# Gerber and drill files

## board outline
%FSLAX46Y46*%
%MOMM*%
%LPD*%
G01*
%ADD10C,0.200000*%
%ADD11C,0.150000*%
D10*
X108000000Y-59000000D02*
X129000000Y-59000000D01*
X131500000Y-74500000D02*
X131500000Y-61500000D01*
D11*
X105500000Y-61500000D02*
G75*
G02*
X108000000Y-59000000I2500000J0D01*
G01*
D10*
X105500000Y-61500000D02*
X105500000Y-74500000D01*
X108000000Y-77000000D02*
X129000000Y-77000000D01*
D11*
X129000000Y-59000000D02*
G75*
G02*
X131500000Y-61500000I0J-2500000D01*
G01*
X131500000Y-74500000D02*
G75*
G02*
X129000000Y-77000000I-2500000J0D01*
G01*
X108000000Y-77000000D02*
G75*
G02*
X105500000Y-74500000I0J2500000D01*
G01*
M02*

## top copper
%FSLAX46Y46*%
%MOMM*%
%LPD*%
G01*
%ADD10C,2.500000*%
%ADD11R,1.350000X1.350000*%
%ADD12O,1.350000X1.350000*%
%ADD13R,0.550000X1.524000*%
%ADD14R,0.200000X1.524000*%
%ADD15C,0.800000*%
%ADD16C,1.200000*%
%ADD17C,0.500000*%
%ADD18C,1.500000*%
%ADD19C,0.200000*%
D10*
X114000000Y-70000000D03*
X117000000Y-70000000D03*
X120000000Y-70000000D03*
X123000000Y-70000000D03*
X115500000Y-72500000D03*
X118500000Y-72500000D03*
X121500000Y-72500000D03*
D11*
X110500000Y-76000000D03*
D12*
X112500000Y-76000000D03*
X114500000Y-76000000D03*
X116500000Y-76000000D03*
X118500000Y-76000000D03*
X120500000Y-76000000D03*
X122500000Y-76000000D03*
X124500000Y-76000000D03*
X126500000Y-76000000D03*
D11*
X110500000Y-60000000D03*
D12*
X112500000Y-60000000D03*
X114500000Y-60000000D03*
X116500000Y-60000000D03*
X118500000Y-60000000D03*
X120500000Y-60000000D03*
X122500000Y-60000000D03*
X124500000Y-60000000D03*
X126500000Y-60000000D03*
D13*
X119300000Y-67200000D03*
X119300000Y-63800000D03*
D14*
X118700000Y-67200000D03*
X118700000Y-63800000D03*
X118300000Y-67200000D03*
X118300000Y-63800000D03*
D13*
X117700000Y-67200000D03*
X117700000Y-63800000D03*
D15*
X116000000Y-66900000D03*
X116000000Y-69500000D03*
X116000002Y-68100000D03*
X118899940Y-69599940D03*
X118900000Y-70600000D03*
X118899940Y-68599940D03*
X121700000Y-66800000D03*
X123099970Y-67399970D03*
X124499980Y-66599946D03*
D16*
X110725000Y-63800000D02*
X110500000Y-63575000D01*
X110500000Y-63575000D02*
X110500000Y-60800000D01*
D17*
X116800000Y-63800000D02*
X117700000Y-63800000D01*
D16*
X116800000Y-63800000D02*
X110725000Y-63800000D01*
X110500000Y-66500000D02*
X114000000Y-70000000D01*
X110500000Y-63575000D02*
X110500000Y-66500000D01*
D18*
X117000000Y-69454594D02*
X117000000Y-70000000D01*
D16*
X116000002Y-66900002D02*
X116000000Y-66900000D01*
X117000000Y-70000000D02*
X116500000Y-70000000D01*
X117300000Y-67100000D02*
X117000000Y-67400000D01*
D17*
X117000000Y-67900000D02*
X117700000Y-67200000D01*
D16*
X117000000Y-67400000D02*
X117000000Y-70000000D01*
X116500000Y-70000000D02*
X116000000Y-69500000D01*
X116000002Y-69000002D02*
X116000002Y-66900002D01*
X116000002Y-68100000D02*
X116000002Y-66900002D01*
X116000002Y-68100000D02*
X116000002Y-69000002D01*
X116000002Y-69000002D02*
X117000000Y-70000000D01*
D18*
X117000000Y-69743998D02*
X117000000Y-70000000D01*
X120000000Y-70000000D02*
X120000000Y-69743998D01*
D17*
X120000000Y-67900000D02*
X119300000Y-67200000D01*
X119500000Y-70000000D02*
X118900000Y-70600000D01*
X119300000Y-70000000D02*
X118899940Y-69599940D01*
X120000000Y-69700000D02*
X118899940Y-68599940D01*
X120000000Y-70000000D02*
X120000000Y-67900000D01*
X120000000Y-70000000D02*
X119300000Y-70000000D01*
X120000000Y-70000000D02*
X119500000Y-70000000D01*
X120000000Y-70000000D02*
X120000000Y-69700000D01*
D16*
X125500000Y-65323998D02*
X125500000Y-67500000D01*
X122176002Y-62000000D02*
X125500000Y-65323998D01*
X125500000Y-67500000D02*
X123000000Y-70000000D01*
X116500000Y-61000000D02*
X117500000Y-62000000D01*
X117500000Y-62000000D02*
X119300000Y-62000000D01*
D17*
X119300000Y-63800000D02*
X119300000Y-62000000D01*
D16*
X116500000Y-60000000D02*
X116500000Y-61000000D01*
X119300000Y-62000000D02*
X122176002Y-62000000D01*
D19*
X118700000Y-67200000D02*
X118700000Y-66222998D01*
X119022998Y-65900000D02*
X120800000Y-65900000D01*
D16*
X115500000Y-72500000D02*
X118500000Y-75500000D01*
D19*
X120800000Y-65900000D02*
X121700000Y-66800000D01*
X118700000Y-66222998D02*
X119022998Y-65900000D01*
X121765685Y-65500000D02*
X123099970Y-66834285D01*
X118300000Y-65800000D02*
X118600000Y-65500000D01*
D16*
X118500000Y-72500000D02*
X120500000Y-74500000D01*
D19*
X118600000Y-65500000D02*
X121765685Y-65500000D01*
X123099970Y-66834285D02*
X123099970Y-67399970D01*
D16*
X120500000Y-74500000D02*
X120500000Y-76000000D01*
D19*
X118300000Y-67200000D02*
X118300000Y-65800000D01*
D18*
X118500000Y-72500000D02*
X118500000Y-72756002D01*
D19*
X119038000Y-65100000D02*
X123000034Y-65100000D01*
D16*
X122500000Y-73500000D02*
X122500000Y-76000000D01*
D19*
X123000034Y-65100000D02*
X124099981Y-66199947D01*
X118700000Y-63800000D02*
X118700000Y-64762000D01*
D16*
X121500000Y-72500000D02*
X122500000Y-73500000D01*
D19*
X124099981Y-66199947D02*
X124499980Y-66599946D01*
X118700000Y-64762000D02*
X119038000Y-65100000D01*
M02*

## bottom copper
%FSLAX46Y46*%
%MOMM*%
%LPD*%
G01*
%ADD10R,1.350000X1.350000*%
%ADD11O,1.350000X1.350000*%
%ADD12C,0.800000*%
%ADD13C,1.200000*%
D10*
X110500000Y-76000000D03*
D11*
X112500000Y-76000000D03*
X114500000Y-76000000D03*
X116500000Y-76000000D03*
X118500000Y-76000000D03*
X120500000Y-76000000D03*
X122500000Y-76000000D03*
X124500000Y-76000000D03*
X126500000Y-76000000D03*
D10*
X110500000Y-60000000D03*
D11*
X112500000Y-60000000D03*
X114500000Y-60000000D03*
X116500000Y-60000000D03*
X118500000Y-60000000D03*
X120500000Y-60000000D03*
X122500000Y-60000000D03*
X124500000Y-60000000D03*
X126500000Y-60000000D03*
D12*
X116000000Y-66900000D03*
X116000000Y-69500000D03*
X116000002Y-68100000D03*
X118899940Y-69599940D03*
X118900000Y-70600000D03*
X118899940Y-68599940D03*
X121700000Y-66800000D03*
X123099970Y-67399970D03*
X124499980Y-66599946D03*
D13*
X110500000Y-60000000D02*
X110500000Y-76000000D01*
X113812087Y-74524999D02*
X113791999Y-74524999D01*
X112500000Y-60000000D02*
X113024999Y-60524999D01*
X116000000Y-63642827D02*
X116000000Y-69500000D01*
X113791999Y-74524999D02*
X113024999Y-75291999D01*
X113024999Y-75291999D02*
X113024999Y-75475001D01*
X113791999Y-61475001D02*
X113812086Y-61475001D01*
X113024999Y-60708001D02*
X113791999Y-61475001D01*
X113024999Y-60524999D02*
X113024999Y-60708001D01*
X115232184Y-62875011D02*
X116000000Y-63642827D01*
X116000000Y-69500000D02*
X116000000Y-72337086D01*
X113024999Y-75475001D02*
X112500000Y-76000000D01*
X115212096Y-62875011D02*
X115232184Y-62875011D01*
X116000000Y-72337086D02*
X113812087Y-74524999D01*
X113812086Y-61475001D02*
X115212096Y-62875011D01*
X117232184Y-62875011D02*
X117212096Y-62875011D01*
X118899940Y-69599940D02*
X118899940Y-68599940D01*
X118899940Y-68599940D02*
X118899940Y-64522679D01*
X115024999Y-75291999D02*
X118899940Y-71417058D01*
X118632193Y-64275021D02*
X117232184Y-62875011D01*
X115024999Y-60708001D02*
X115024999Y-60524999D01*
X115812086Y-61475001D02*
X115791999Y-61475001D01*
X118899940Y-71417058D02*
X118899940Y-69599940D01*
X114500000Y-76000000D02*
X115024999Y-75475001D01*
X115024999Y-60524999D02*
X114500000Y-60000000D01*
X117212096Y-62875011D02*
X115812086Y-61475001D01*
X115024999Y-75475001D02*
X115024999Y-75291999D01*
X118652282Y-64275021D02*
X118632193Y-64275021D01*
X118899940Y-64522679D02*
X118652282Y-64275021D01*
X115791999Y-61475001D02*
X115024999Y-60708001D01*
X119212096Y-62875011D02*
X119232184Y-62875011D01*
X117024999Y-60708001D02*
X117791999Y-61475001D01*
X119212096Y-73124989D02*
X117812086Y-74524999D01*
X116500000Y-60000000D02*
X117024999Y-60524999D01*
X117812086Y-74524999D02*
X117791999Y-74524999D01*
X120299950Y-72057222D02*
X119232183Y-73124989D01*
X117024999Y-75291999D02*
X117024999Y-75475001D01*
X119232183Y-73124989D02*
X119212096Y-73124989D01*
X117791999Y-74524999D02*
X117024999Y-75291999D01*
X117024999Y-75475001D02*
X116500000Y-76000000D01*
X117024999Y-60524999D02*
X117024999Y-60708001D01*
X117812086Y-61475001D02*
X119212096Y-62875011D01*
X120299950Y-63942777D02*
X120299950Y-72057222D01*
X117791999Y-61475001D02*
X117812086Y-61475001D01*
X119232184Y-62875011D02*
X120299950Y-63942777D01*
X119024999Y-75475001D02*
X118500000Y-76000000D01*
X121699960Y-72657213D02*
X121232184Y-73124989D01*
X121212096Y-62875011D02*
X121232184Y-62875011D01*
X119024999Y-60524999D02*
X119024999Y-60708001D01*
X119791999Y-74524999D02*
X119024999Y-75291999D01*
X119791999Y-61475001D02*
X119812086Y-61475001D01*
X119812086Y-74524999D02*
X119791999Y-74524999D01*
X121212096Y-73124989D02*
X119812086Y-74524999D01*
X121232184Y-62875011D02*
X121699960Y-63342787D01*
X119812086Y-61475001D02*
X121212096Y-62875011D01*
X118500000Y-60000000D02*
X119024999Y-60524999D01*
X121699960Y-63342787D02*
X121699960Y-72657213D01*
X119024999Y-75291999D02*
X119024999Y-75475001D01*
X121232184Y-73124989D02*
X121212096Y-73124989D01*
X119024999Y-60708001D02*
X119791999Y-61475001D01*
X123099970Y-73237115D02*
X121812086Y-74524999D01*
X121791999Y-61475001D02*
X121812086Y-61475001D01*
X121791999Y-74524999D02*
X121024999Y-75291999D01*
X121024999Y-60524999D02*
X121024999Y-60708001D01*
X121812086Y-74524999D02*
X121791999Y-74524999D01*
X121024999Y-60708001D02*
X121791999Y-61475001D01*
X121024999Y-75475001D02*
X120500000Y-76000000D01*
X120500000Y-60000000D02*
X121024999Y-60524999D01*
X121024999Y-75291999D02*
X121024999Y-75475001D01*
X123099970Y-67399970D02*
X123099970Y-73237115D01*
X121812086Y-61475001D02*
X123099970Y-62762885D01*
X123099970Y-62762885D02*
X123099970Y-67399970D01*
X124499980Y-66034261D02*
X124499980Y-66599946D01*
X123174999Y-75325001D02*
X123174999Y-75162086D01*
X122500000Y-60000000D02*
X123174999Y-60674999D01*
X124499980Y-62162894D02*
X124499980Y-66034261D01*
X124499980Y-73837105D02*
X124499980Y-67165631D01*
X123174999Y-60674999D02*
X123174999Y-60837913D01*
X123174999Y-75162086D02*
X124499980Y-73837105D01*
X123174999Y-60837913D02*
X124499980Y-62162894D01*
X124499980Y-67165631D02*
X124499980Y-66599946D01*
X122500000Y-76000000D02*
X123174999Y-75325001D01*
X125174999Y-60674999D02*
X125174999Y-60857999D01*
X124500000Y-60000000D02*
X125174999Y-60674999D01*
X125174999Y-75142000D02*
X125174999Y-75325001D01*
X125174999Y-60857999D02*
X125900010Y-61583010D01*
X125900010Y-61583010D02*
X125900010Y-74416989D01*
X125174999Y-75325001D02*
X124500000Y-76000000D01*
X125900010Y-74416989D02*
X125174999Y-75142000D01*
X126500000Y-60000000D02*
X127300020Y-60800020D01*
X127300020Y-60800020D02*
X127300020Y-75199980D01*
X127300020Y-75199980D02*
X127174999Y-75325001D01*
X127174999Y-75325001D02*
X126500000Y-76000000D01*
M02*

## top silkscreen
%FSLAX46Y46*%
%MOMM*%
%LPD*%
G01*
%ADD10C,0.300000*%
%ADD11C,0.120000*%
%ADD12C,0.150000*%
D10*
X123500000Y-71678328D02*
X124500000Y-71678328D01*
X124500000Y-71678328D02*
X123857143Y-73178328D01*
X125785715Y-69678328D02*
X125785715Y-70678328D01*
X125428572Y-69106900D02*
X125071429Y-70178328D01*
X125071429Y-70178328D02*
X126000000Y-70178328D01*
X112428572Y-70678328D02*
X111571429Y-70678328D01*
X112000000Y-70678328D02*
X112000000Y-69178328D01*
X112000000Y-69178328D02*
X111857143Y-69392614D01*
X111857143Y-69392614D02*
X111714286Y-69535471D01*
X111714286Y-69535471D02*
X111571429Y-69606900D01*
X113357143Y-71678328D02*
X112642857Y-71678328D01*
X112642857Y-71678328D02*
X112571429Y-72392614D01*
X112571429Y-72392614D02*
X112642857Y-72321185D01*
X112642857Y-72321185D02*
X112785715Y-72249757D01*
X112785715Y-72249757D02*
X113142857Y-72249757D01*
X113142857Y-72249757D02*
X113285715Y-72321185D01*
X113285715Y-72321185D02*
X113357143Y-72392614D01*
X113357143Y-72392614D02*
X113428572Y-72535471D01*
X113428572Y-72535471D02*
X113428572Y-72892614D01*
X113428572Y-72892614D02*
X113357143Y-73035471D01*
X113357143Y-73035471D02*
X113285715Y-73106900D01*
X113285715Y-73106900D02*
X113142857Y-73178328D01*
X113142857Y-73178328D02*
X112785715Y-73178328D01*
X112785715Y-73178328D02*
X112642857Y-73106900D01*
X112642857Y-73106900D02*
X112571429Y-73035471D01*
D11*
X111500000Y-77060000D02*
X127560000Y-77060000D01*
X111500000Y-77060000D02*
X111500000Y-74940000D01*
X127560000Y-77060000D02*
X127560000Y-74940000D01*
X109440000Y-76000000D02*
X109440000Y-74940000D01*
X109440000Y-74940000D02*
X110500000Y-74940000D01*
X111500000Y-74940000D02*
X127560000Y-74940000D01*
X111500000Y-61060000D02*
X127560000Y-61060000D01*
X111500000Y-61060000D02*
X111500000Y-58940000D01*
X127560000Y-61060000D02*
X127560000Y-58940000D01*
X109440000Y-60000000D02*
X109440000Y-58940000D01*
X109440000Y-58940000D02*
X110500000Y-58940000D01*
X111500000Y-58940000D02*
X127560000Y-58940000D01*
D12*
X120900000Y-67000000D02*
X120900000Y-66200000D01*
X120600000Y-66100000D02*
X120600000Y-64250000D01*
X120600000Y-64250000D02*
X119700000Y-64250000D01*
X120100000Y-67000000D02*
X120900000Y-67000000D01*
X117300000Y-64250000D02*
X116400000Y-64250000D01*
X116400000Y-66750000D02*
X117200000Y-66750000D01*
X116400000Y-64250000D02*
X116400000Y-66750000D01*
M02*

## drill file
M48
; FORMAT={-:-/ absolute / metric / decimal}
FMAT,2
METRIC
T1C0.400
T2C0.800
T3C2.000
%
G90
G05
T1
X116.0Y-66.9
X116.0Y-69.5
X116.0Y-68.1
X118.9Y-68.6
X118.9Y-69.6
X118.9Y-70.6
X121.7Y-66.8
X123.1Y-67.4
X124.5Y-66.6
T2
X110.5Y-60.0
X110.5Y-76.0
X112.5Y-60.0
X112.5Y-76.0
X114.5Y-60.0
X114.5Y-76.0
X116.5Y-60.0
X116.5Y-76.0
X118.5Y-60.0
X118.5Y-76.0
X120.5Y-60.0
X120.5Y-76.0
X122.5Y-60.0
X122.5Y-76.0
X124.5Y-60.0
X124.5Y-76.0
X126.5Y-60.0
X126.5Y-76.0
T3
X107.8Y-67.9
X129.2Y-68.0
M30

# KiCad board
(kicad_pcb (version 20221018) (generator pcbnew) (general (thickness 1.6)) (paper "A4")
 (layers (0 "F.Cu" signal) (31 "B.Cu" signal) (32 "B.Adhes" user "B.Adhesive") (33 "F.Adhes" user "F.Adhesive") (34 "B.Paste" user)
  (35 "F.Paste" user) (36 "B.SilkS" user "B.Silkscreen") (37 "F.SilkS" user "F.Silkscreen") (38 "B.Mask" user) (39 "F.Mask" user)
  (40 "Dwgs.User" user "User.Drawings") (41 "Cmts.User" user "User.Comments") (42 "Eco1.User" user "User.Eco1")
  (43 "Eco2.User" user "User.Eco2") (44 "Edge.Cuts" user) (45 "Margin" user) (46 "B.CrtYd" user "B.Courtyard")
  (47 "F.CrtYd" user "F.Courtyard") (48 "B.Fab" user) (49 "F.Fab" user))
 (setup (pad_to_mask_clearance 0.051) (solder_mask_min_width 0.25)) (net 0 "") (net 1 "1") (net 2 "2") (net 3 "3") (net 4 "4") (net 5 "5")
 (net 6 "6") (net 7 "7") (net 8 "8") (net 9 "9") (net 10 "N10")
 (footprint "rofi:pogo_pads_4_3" (layer "F.Cu") (at 118.5 70)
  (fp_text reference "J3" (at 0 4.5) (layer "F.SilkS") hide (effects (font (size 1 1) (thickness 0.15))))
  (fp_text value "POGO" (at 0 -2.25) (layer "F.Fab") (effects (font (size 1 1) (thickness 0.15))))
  (pad "1" smd circle (at -4.5 0) (size 2.5 2.5) (layers "F.Cu" "F.Paste" "F.Mask") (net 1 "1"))
  (pad "2" smd circle (at -1.5 0) (size 2.5 2.5) (layers "F.Cu" "F.Paste" "F.Mask") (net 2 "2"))
  (pad "3" smd circle (at 1.5 0) (size 2.5 2.5) (layers "F.Cu" "F.Paste" "F.Mask") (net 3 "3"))
  (pad "4" smd circle (at 4.5 0) (size 2.5 2.5) (layers "F.Cu" "F.Paste" "F.Mask") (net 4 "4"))
  (pad "5" smd circle (at -3 2.5) (size 2.5 2.5) (layers "F.Cu" "F.Paste" "F.Mask") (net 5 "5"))
  (pad "6" smd circle (at 0 2.5) (size 2.5 2.5) (layers "F.Cu" "F.Paste" "F.Mask") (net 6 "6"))
  (pad "7" smd circle (at 3 2.5) (size 2.5 2.5) (layers "F.Cu" "F.Paste" "F.Mask") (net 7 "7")))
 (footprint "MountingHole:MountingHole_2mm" (layer "F.Cu") (at 129.2 68)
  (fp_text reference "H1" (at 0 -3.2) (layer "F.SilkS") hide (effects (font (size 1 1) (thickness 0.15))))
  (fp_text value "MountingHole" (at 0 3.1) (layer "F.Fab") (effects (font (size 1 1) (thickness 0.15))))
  (pad "" np_thru_hole circle (at 0 0) (size 2 2) (drill 2) (layers "*.Cu" "*.Mask")))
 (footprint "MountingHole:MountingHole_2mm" (layer "F.Cu") (at 107.8 67.9)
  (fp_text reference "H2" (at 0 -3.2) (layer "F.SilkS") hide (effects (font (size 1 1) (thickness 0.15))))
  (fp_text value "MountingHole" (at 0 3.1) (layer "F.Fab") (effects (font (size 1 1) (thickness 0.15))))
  (pad "" np_thru_hole circle (at 0 0) (size 2 2) (drill 2) (layers "*.Cu" "*.Mask")))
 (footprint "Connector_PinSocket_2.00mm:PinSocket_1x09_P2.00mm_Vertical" (layer "F.Cu") (at 110.5 76 90)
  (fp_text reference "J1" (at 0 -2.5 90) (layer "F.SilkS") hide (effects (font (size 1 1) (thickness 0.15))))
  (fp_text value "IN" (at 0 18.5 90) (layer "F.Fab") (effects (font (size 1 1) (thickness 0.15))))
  (fp_line (start -1.06 1) (end -1.06 17.06) (stroke (width 0.12) (type solid)) (layer "F.SilkS"))
  (fp_line (start -1.06 1) (end 1.06 1) (stroke (width 0.12) (type solid)) (layer "F.SilkS"))
  (fp_line (start -1.06 17.06) (end 1.06 17.06) (stroke (width 0.12) (type solid)) (layer "F.SilkS"))
  (fp_line (start 0 -1.06) (end 1.06 -1.06) (stroke (width 0.12) (type solid)) (layer "F.SilkS"))
  (fp_line (start 1.06 -1.06) (end 1.06 0) (stroke (width 0.12) (type solid)) (layer "F.SilkS"))
  (fp_line (start 1.06 1) (end 1.06 17.06) (stroke (width 0.12) (type solid)) (layer "F.SilkS"))
  (pad "1" thru_hole rect (at 0 0 90) (size 1.35 1.35) (drill 0.8) (layers "*.Cu" "*.Mask") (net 1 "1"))
  (pad "2" thru_hole oval (at 0 2 90) (size 1.35 1.35) (drill 0.8) (layers "*.Cu" "*.Mask") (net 2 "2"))
  (pad "3" thru_hole oval (at 0 4 90) (size 1.35 1.35) (drill 0.8) (layers "*.Cu" "*.Mask") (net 3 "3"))
  (pad "4" thru_hole oval (at 0 6 90) (size 1.35 1.35) (drill 0.8) (layers "*.Cu" "*.Mask") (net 4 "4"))
  (pad "5" thru_hole oval (at 0 8 90) (size 1.35 1.35) (drill 0.8) (layers "*.Cu" "*.Mask") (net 5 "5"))
  (pad "6" thru_hole oval (at 0 10 90) (size 1.35 1.35) (drill 0.8) (layers "*.Cu" "*.Mask") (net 6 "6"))
  (pad "7" thru_hole oval (at 0 12 90) (size 1.35 1.35) (drill 0.8) (layers "*.Cu" "*.Mask") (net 7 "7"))
  (pad "8" thru_hole oval (at 0 14 90) (size 1.35 1.35) (drill 0.8) (layers "*.Cu" "*.Mask") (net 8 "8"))
  (pad "9" thru_hole oval (at 0 16 90) (size 1.35 1.35) (drill 0.8) (layers "*.Cu" "*.Mask") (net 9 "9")))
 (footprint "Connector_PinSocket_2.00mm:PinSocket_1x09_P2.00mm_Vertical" (layer "F.Cu") (at 110.5 60 90)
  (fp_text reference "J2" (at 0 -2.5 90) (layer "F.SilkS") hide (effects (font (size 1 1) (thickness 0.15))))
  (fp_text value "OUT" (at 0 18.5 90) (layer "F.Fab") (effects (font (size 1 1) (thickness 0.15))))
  (fp_line (start -1.06 1) (end -1.06 17.06) (stroke (width 0.12) (type solid)) (layer "F.SilkS"))
  (fp_line (start -1.06 1) (end 1.06 1) (stroke (width 0.12) (type solid)) (layer "F.SilkS"))
  (fp_line (start -1.06 17.06) (end 1.06 17.06) (stroke (width 0.12) (type solid)) (layer "F.SilkS"))
  (fp_line (start 0 -1.06) (end 1.06 -1.06) (stroke (width 0.12) (type solid)) (layer "F.SilkS"))
  (fp_line (start 1.06 -1.06) (end 1.06 0) (stroke (width 0.12) (type solid)) (layer "F.SilkS"))
  (fp_line (start 1.06 1) (end 1.06 17.06) (stroke (width 0.12) (type solid)) (layer "F.SilkS"))
  (pad "1" thru_hole rect (at 0 0 90) (size 1.35 1.35) (drill 0.8) (layers "*.Cu" "*.Mask") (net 1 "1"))
  (pad "2" thru_hole oval (at 0 2 90) (size 1.35 1.35) (drill 0.8) (layers "*.Cu" "*.Mask") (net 2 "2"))
  (pad "3" thru_hole oval (at 0 4 90) (size 1.35 1.35) (drill 0.8) (layers "*.Cu" "*.Mask") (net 3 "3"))
  (pad "4" thru_hole oval (at 0 6 90) (size 1.35 1.35) (drill 0.8) (layers "*.Cu" "*.Mask") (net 4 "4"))
  (pad "5" thru_hole oval (at 0 8 90) (size 1.35 1.35) (drill 0.8) (layers "*.Cu" "*.Mask") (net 5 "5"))
  (pad "6" thru_hole oval (at 0 10 90) (size 1.35 1.35) (drill 0.8) (layers "*.Cu" "*.Mask") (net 6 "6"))
  (pad "7" thru_hole oval (at 0 12 90) (size 1.35 1.35) (drill 0.8) (layers "*.Cu" "*.Mask") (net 7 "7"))
  (pad "8" thru_hole oval (at 0 14 90) (size 1.35 1.35) (drill 0.8) (layers "*.Cu" "*.Mask") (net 8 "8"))
  (pad "9" thru_hole oval (at 0 16 90) (size 1.35 1.35) (drill 0.8) (layers "*.Cu" "*.Mask") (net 9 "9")))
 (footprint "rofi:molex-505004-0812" (layer "F.Cu") (at 118.5 65.5 180)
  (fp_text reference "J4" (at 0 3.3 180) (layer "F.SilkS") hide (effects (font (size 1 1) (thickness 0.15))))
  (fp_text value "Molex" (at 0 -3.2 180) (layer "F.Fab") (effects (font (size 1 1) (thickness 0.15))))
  (fp_line (start -2.4 -1.5) (end -2.4 -0.7) (stroke (width 0.15) (type solid)) (layer "F.SilkS"))
  (fp_line (start -2.1 -0.6) (end -2.1 1.25) (stroke (width 0.15) (type solid)) (layer "F.SilkS"))
  (fp_line (start -2.1 1.25) (end -1.2 1.25) (stroke (width 0.15) (type solid)) (layer "F.SilkS"))
  (fp_line (start -1.6 -1.5) (end -2.4 -1.5) (stroke (width 0.15) (type solid)) (layer "F.SilkS"))
  (fp_line (start 1.2 1.25) (end 2.1 1.25) (stroke (width 0.15) (type solid)) (layer "F.SilkS"))
  (fp_line (start 2.1 -1.25) (end 1.3 -1.25) (stroke (width 0.15) (type solid)) (layer "F.SilkS"))
  (fp_line (start 2.1 1.25) (end 2.1 -1.25) (stroke (width 0.15) (type solid)) (layer "F.SilkS"))
  (pad "1" smd rect (at -0.8 -1.7 180) (size 0.55 1.524) (layers "F.Cu" "F.Paste" "F.Mask") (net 3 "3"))
  (pad "2" smd rect (at -0.8 1.7 180) (size 0.55 1.524) (layers "F.Cu" "F.Paste" "F.Mask") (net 4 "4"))
  (pad "3" smd rect (at -0.2 -1.7 180) (size 0.2 1.524) (layers "F.Cu" "F.Paste" "F.Mask") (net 5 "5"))
  (pad "4" smd rect (at -0.2 1.7 180) (size 0.2 1.524) (layers "F.Cu" "F.Paste" "F.Mask") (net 7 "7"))
  (pad "5" smd rect (at 0.2 -1.7 180) (size 0.2 1.524) (layers "F.Cu" "F.Paste" "F.Mask") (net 6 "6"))
  (pad "6" smd rect (at 0.2 1.7 180) (size 0.2 1.524) (layers "F.Cu" "F.Paste" "F.Mask") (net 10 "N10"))
  (pad "7" smd rect (at 0.8 -1.7 180) (size 0.55 1.524) (layers "F.Cu" "F.Paste" "F.Mask") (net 2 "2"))
  (pad "8" smd rect (at 0.8 1.7 180) (size 0.55 1.524) (layers "F.Cu" "F.Paste" "F.Mask") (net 1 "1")))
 (gr_line (start 108 59) (end 129 59) (stroke (width 0.2) (type solid)) (layer "Edge.Cuts"))
 (gr_line (start 131.5 74.5) (end 131.5 61.5) (stroke (width 0.2) (type solid)) (layer "Edge.Cuts"))
 (gr_arc (start 105.5 61.5) (mid 106.232233 59.732233) (end 108 59) (stroke (width 0.15) (type solid)) (layer "Edge.Cuts"))
 (gr_line (start 105.5 61.5) (end 105.5 74.5) (stroke (width 0.2) (type solid)) (layer "Edge.Cuts"))
 (gr_line (start 108 77) (end 129 77) (stroke (width 0.2) (type solid)) (layer "Edge.Cuts"))
 (gr_arc (start 129 59) (mid 130.767767 59.732233) (end 131.5 61.5) (stroke (width 0.15) (type solid)) (layer "Edge.Cuts"))
 (gr_arc (start 131.5 74.5) (mid 130.767767 76.267767) (end 129 77) (stroke (width 0.15) (type solid)) (layer "Edge.Cuts"))
 (gr_arc (start 108 77) (mid 106.232233 76.267767) (end 105.5 74.5) (stroke (width 0.15) (type solid)) (layer "Edge.Cuts"))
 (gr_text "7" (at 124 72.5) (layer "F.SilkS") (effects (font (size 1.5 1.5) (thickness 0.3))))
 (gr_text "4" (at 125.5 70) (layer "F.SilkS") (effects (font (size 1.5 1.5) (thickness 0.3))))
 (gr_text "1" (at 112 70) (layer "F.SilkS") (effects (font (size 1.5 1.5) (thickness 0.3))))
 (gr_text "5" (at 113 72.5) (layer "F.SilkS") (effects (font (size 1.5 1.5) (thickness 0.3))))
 (segment (start 110.725 63.8) (end 110.5 63.575) (width 1.2) (layer "F.Cu") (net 1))
 (segment (start 110.5 63.575) (end 110.5 60.8) (width 1.2) (layer "F.Cu") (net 1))
 (segment (start 116.8 63.8) (end 117.7 63.8) (width 0.5) (layer "F.Cu") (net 1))
 (segment (start 116.8 63.8) (end 110.725 63.8) (width 1.2) (layer "F.Cu") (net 1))
 (segment (start 110.5 66.5) (end 114 70) (width 1.2) (layer "F.Cu") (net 1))
 (segment (start 110.5 63.575) (end 110.5 66.5) (width 1.2) (layer "F.Cu") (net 1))
 (segment (start 110.5 60) (end 110.5 76) (width 1.2) (layer "B.Cu") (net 1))
 (segment (start 117 69.454594) (end 117 70) (width 1.5) (layer "F.Cu") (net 2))
 (segment (start 116.000002 66.900002) (end 116 66.9) (width 1.2) (layer "F.Cu") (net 2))
 (segment (start 117 70) (end 116.5 70) (width 1.2) (layer "F.Cu") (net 2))
 (segment (start 117.3 67.1) (end 117 67.4) (width 1.2) (layer "F.Cu") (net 2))
 (segment (start 117 67.9) (end 117.7 67.2) (width 0.5) (layer "F.Cu") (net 2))
 (segment (start 117 67.4) (end 117 70) (width 1.2) (layer "F.Cu") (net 2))
 (segment (start 116.5 70) (end 116 69.5) (width 1.2) (layer "F.Cu") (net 2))
 (segment (start 116.000002 69.000002) (end 116.000002 66.900002) (width 1.2) (layer "F.Cu") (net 2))
 (segment (start 116.000002 68.1) (end 116.000002 66.900002) (width 1.2) (layer "F.Cu") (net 2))
 (segment (start 116.000002 68.1) (end 116.000002 69.000002) (width 1.2) (layer "F.Cu") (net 2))
 (segment (start 116.000002 69.000002) (end 117 70) (width 1.2) (layer "F.Cu") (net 2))
 (segment (start 117 69.743998) (end 117 70) (width 1.5) (layer "F.Cu") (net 2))
 (via (at 116 66.9) (size 0.8) (drill 0.4) (layers "F.Cu" "B.Cu") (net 2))
 (via (at 116 69.5) (size 0.8) (drill 0.4) (layers "F.Cu" "B.Cu") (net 2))
 (via (at 116.000002 68.1) (size 0.8) (drill 0.4) (layers "F.Cu" "B.Cu") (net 2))
 (segment (start 113.812087 74.524999) (end 113.791999 74.524999) (width 1.2) (layer "B.Cu") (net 2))
 (segment (start 112.5 60) (end 113.024999 60.524999) (width 1.2) (layer "B.Cu") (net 2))
 (segment (start 116 63.642827) (end 116 69.5) (width 1.2) (layer "B.Cu") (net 2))
 (segment (start 113.791999 74.524999) (end 113.024999 75.291999) (width 1.2) (layer "B.Cu") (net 2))
 (segment (start 113.024999 75.291999) (end 113.024999 75.475001) (width 1.2) (layer "B.Cu") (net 2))
 (segment (start 113.791999 61.475001) (end 113.812086 61.475001) (width 1.2) (layer "B.Cu") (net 2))
 (segment (start 113.024999 60.708001) (end 113.791999 61.475001) (width 1.2) (layer "B.Cu") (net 2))
 (segment (start 113.024999 60.524999) (end 113.024999 60.708001) (width 1.2) (layer "B.Cu") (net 2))
 (segment (start 115.232184 62.875011) (end 116 63.642827) (width 1.2) (layer "B.Cu") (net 2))
 (segment (start 116 69.5) (end 116 72.337086) (width 1.2) (layer "B.Cu") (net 2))
 (segment (start 113.024999 75.475001) (end 112.5 76) (width 1.2) (layer "B.Cu") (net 2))
 (segment (start 115.212096 62.875011) (end 115.232184 62.875011) (width 1.2) (layer "B.Cu") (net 2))
 (segment (start 116 72.337086) (end 113.812087 74.524999) (width 1.2) (layer "B.Cu") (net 2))
 (segment (start 113.812086 61.475001) (end 115.212096 62.875011) (width 1.2) (layer "B.Cu") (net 2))
 (segment (start 120 70) (end 120 69.743998) (width 1.5) (layer "F.Cu") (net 3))
 (segment (start 120 67.9) (end 119.3 67.2) (width 0.5) (layer "F.Cu") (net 3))
 (segment (start 119.5 70) (end 118.9 70.6) (width 0.5) (layer "F.Cu") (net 3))
 (segment (start 119.3 70) (end 118.89994 69.59994) (width 0.5) (layer "F.Cu") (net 3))
 (segment (start 120 69.7) (end 118.89994 68.59994) (width 0.5) (layer "F.Cu") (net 3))
 (segment (start 120 70) (end 120 67.9) (width 0.5) (layer "F.Cu") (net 3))
 (segment (start 120 70) (end 119.3 70) (width 0.5) (layer "F.Cu") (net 3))
 (segment (start 120 70) (end 119.5 70) (width 0.5) (layer "F.Cu") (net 3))
 (segment (start 120 70) (end 120 69.7) (width 0.5) (layer "F.Cu") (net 3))
 (via (at 118.89994 69.59994) (size 0.8) (drill 0.4) (layers "F.Cu" "B.Cu") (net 3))
 (via (at 118.9 70.6) (size 0.8) (drill 0.4) (layers "F.Cu" "B.Cu") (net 3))
 (via (at 118.89994 68.59994) (size 0.8) (drill 0.4) (layers "F.Cu" "B.Cu") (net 3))
 (segment (start 117.232184 62.875011) (end 117.212096 62.875011) (width 1.2) (layer "B.Cu") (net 3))
 (segment (start 118.89994 69.59994) (end 118.89994 68.59994) (width 1.2) (layer "B.Cu") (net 3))
 (segment (start 118.89994 68.59994) (end 118.89994 64.522679) (width 1.2) (layer "B.Cu") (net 3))
 (segment (start 115.024999 75.291999) (end 118.89994 71.417058) (width 1.2) (layer "B.Cu") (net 3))
 (segment (start 118.632193 64.275021) (end 117.232184 62.875011) (width 1.2) (layer "B.Cu") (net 3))
 (segment (start 115.024999 60.708001) (end 115.024999 60.524999) (width 1.2) (layer "B.Cu") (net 3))
 (segment (start 115.812086 61.475001) (end 115.791999 61.475001) (width 1.2) (layer "B.Cu") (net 3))
 (segment (start 118.89994 71.417058) (end 118.89994 69.59994) (width 1.2) (layer "B.Cu") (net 3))
 (segment (start 114.5 76) (end 115.024999 75.475001) (width 1.2) (layer "B.Cu") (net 3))
 (segment (start 115.024999 60.524999) (end 114.5 60) (width 1.2) (layer "B.Cu") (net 3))
 (segment (start 117.212096 62.875011) (end 115.812086 61.475001) (width 1.2) (layer "B.Cu") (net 3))
 (segment (start 115.024999 75.475001) (end 115.024999 75.291999) (width 1.2) (layer "B.Cu") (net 3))
 (segment (start 118.652282 64.275021) (end 118.632193 64.275021) (width 1.2) (layer "B.Cu") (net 3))
 (segment (start 118.89994 64.522679) (end 118.652282 64.275021) (width 1.2) (layer "B.Cu") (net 3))
 (segment (start 115.791999 61.475001) (end 115.024999 60.708001) (width 1.2) (layer "B.Cu") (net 3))
 (segment (start 125.5 65.323998) (end 125.5 67.5) (width 1.2) (layer "F.Cu") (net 4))
 (segment (start 122.176002 62) (end 125.5 65.323998) (width 1.2) (layer "F.Cu") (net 4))
 (segment (start 125.5 67.5) (end 123 70) (width 1.2) (layer "F.Cu") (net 4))
 (segment (start 116.5 61) (end 117.5 62) (width 1.2) (layer "F.Cu") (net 4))
 (segment (start 117.5 62) (end 119.3 62) (width 1.2) (layer "F.Cu") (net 4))
 (segment (start 119.3 63.8) (end 119.3 62) (width 0.5) (layer "F.Cu") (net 4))
 (segment (start 116.5 60) (end 116.5 61) (width 1.2) (layer "F.Cu") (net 4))
 (segment (start 119.3 62) (end 122.176002 62) (width 1.2) (layer "F.Cu") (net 4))
 (segment (start 119.212096 62.875011) (end 119.232184 62.875011) (width 1.2) (layer "B.Cu") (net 4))
 (segment (start 117.024999 60.708001) (end 117.791999 61.475001) (width 1.2) (layer "B.Cu") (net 4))
 (segment (start 119.212096 73.124989) (end 117.812086 74.524999) (width 1.2) (layer "B.Cu") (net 4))
 (segment (start 116.5 60) (end 117.024999 60.524999) (width 1.2) (layer "B.Cu") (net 4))
 (segment (start 117.812086 74.524999) (end 117.791999 74.524999) (width 1.2) (layer "B.Cu") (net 4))
 (segment (start 120.29995 72.057222) (end 119.232183 73.124989) (width 1.2) (layer "B.Cu") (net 4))
 (segment (start 117.024999 75.291999) (end 117.024999 75.475001) (width 1.2) (layer "B.Cu") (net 4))
 (segment (start 119.232183 73.124989) (end 119.212096 73.124989) (width 1.2) (layer "B.Cu") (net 4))
 (segment (start 117.791999 74.524999) (end 117.024999 75.291999) (width 1.2) (layer "B.Cu") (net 4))
 (segment (start 117.024999 75.475001) (end 116.5 76) (width 1.2) (layer "B.Cu") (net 4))
 (segment (start 117.024999 60.524999) (end 117.024999 60.708001) (width 1.2) (layer "B.Cu") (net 4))
 (segment (start 117.812086 61.475001) (end 119.212096 62.875011) (width 1.2) (layer "B.Cu") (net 4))
 (segment (start 120.29995 63.942777) (end 120.29995 72.057222) (width 1.2) (layer "B.Cu") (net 4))
 (segment (start 117.791999 61.475001) (end 117.812086 61.475001) (width 1.2) (layer "B.Cu") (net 4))
 (segment (start 119.232184 62.875011) (end 120.29995 63.942777) (width 1.2) (layer "B.Cu") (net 4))
 (segment (start 118.7 67.2) (end 118.7 66.222998) (width 0.2) (layer "F.Cu") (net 5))
 (segment (start 119.022998 65.9) (end 120.8 65.9) (width 0.2) (layer "F.Cu") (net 5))
 (segment (start 115.5 72.5) (end 118.5 75.5) (width 1.2) (layer "F.Cu") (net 5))
 (segment (start 120.8 65.9) (end 121.7 66.8) (width 0.2) (layer "F.Cu") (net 5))
 (segment (start 118.7 66.222998) (end 119.022998 65.9) (width 0.2) (layer "F.Cu") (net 5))
 (via (at 121.7 66.8) (size 0.8) (drill 0.4) (layers "F.Cu" "B.Cu") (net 5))
 (segment (start 119.024999 75.475001) (end 118.5 76) (width 1.2) (layer "B.Cu") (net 5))
 (segment (start 121.69996 72.657213) (end 121.232184 73.124989) (width 1.2) (layer "B.Cu") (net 5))
 (segment (start 121.212096 62.875011) (end 121.232184 62.875011) (width 1.2) (layer "B.Cu") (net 5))
 (segment (start 119.024999 60.524999) (end 119.024999 60.708001) (width 1.2) (layer "B.Cu") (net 5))
 (segment (start 119.791999 74.524999) (end 119.024999 75.291999) (width 1.2) (layer "B.Cu") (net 5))
 (segment (start 119.791999 61.475001) (end 119.812086 61.475001) (width 1.2) (layer "B.Cu") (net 5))
 (segment (start 119.812086 74.524999) (end 119.791999 74.524999) (width 1.2) (layer "B.Cu") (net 5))
 (segment (start 121.212096 73.124989) (end 119.812086 74.524999) (width 1.2) (layer "B.Cu") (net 5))
 (segment (start 121.232184 62.875011) (end 121.69996 63.342787) (width 1.2) (layer "B.Cu") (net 5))
 (segment (start 119.812086 61.475001) (end 121.212096 62.875011) (width 1.2) (layer "B.Cu") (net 5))
 (segment (start 118.5 60) (end 119.024999 60.524999) (width 1.2) (layer "B.Cu") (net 5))
 (segment (start 121.69996 63.342787) (end 121.69996 72.657213) (width 1.2) (layer "B.Cu") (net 5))
 (segment (start 119.024999 75.291999) (end 119.024999 75.475001) (width 1.2) (layer "B.Cu") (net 5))
 (segment (start 121.232184 73.124989) (end 121.212096 73.124989) (width 1.2) (layer "B.Cu") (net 5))
 (segment (start 119.024999 60.708001) (end 119.791999 61.475001) (width 1.2) (layer "B.Cu") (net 5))
 (segment (start 121.765685 65.5) (end 123.09997 66.834285) (width 0.2) (layer "F.Cu") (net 6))
 (segment (start 118.3 65.8) (end 118.6 65.5) (width 0.2) (layer "F.Cu") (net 6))
 (segment (start 118.5 72.5) (end 120.5 74.5) (width 1.2) (layer "F.Cu") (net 6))
 (segment (start 118.6 65.5) (end 121.765685 65.5) (width 0.2) (layer "F.Cu") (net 6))
 (segment (start 123.09997 66.834285) (end 123.09997 67.39997) (width 0.2) (layer "F.Cu") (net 6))
 (segment (start 120.5 74.5) (end 120.5 76) (width 1.2) (layer "F.Cu") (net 6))
 (segment (start 118.3 67.2) (end 118.3 65.8) (width 0.2) (layer "F.Cu") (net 6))
 (segment (start 118.5 72.5) (end 118.5 72.756002) (width 1.5) (layer "F.Cu") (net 6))
 (via (at 123.09997 67.39997) (size 0.8) (drill 0.4) (layers "F.Cu" "B.Cu") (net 6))
 (segment (start 123.09997 73.237115) (end 121.812086 74.524999) (width 1.2) (layer "B.Cu") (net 6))
 (segment (start 121.791999 61.475001) (end 121.812086 61.475001) (width 1.2) (layer "B.Cu") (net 6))
 (segment (start 121.791999 74.524999) (end 121.024999 75.291999) (width 1.2) (layer "B.Cu") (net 6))
 (segment (start 121.024999 60.524999) (end 121.024999 60.708001) (width 1.2) (layer "B.Cu") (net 6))
 (segment (start 121.812086 74.524999) (end 121.791999 74.524999) (width 1.2) (layer "B.Cu") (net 6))
 (segment (start 121.024999 60.708001) (end 121.791999 61.475001) (width 1.2) (layer "B.Cu") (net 6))
 (segment (start 121.024999 75.475001) (end 120.5 76) (width 1.2) (layer "B.Cu") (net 6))
 (segment (start 120.5 60) (end 121.024999 60.524999) (width 1.2) (layer "B.Cu") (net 6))
 (segment (start 121.024999 75.291999) (end 121.024999 75.475001) (width 1.2) (layer "B.Cu") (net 6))
 (segment (start 123.09997 67.39997) (end 123.09997 73.237115) (width 1.2) (layer "B.Cu") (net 6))
 (segment (start 121.812086 61.475001) (end 123.09997 62.762885) (width 1.2) (layer "B.Cu") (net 6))
 (segment (start 123.09997 62.762885) (end 123.09997 67.39997) (width 1.2) (layer "B.Cu") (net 6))
 (segment (start 119.038 65.1) (end 123.000034 65.1) (width 0.2) (layer "F.Cu") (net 7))
 (segment (start 122.5 73.5) (end 122.5 76) (width 1.2) (layer "F.Cu") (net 7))
 (segment (start 123.000034 65.1) (end 124.099981 66.199947) (width 0.2) (layer "F.Cu") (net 7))
 (segment (start 118.7 63.8) (end 118.7 64.762) (width 0.2) (layer "F.Cu") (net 7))
 (segment (start 121.5 72.5) (end 122.5 73.5) (width 1.2) (layer "F.Cu") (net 7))
 (segment (start 124.099981 66.199947) (end 124.49998 66.599946) (width 0.2) (layer "F.Cu") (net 7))
 (segment (start 118.7 64.762) (end 119.038 65.1) (width 0.2) (layer "F.Cu") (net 7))
 (via (at 124.49998 66.599946) (size 0.8) (drill 0.4) (layers "F.Cu" "B.Cu") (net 7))
 (segment (start 124.49998 66.034261) (end 124.49998 66.599946) (width 1.2) (layer "B.Cu") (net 7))
 (segment (start 123.174999 75.325001) (end 123.174999 75.162086) (width 1.2) (layer "B.Cu") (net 7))
 (segment (start 122.5 60) (end 123.174999 60.674999) (width 1.2) (layer "B.Cu") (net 7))
 (segment (start 124.49998 62.162894) (end 124.49998 66.034261) (width 1.2) (layer "B.Cu") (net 7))
 (segment (start 124.49998 73.837105) (end 124.49998 67.165631) (width 1.2) (layer "B.Cu") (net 7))
 (segment (start 123.174999 60.674999) (end 123.174999 60.837913) (width 1.2) (layer "B.Cu") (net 7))
 (segment (start 123.174999 75.162086) (end 124.49998 73.837105) (width 1.2) (layer "B.Cu") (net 7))
 (segment (start 123.174999 60.837913) (end 124.49998 62.162894) (width 1.2) (layer "B.Cu") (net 7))
 (segment (start 124.49998 67.165631) (end 124.49998 66.599946) (width 1.2) (layer "B.Cu") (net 7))
 (segment (start 122.5 76) (end 123.174999 75.325001) (width 1.2) (layer "B.Cu") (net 7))
 (segment (start 125.174999 60.674999) (end 125.174999 60.857999) (width 1.2) (layer "B.Cu") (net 8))
 (segment (start 124.5 60) (end 125.174999 60.674999) (width 1.2) (layer "B.Cu") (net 8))
 (segment (start 125.174999 75.142) (end 125.174999 75.325001) (width 1.2) (layer "B.Cu") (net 8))
 (segment (start 125.174999 60.857999) (end 125.90001 61.58301) (width 1.2) (layer "B.Cu") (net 8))
 (segment (start 125.90001 61.58301) (end 125.90001 74.416989) (width 1.2) (layer "B.Cu") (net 8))
 (segment (start 125.174999 75.325001) (end 124.5 76) (width 1.2) (layer "B.Cu") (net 8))
 (segment (start 125.90001 74.416989) (end 125.174999 75.142) (width 1.2) (layer "B.Cu") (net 8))
 (segment (start 126.5 60) (end 127.30002 60.80002) (width 1.2) (layer "B.Cu") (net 9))
 (segment (start 127.30002 60.80002) (end 127.30002 75.19998) (width 1.2) (layer "B.Cu") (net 9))
 (segment (start 127.30002 75.19998) (end 127.174999 75.325001) (width 1.2) (layer "B.Cu") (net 9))
 (segment (start 127.174999 75.325001) (end 126.5 76) (width 1.2) (layer "B.Cu") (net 9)))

